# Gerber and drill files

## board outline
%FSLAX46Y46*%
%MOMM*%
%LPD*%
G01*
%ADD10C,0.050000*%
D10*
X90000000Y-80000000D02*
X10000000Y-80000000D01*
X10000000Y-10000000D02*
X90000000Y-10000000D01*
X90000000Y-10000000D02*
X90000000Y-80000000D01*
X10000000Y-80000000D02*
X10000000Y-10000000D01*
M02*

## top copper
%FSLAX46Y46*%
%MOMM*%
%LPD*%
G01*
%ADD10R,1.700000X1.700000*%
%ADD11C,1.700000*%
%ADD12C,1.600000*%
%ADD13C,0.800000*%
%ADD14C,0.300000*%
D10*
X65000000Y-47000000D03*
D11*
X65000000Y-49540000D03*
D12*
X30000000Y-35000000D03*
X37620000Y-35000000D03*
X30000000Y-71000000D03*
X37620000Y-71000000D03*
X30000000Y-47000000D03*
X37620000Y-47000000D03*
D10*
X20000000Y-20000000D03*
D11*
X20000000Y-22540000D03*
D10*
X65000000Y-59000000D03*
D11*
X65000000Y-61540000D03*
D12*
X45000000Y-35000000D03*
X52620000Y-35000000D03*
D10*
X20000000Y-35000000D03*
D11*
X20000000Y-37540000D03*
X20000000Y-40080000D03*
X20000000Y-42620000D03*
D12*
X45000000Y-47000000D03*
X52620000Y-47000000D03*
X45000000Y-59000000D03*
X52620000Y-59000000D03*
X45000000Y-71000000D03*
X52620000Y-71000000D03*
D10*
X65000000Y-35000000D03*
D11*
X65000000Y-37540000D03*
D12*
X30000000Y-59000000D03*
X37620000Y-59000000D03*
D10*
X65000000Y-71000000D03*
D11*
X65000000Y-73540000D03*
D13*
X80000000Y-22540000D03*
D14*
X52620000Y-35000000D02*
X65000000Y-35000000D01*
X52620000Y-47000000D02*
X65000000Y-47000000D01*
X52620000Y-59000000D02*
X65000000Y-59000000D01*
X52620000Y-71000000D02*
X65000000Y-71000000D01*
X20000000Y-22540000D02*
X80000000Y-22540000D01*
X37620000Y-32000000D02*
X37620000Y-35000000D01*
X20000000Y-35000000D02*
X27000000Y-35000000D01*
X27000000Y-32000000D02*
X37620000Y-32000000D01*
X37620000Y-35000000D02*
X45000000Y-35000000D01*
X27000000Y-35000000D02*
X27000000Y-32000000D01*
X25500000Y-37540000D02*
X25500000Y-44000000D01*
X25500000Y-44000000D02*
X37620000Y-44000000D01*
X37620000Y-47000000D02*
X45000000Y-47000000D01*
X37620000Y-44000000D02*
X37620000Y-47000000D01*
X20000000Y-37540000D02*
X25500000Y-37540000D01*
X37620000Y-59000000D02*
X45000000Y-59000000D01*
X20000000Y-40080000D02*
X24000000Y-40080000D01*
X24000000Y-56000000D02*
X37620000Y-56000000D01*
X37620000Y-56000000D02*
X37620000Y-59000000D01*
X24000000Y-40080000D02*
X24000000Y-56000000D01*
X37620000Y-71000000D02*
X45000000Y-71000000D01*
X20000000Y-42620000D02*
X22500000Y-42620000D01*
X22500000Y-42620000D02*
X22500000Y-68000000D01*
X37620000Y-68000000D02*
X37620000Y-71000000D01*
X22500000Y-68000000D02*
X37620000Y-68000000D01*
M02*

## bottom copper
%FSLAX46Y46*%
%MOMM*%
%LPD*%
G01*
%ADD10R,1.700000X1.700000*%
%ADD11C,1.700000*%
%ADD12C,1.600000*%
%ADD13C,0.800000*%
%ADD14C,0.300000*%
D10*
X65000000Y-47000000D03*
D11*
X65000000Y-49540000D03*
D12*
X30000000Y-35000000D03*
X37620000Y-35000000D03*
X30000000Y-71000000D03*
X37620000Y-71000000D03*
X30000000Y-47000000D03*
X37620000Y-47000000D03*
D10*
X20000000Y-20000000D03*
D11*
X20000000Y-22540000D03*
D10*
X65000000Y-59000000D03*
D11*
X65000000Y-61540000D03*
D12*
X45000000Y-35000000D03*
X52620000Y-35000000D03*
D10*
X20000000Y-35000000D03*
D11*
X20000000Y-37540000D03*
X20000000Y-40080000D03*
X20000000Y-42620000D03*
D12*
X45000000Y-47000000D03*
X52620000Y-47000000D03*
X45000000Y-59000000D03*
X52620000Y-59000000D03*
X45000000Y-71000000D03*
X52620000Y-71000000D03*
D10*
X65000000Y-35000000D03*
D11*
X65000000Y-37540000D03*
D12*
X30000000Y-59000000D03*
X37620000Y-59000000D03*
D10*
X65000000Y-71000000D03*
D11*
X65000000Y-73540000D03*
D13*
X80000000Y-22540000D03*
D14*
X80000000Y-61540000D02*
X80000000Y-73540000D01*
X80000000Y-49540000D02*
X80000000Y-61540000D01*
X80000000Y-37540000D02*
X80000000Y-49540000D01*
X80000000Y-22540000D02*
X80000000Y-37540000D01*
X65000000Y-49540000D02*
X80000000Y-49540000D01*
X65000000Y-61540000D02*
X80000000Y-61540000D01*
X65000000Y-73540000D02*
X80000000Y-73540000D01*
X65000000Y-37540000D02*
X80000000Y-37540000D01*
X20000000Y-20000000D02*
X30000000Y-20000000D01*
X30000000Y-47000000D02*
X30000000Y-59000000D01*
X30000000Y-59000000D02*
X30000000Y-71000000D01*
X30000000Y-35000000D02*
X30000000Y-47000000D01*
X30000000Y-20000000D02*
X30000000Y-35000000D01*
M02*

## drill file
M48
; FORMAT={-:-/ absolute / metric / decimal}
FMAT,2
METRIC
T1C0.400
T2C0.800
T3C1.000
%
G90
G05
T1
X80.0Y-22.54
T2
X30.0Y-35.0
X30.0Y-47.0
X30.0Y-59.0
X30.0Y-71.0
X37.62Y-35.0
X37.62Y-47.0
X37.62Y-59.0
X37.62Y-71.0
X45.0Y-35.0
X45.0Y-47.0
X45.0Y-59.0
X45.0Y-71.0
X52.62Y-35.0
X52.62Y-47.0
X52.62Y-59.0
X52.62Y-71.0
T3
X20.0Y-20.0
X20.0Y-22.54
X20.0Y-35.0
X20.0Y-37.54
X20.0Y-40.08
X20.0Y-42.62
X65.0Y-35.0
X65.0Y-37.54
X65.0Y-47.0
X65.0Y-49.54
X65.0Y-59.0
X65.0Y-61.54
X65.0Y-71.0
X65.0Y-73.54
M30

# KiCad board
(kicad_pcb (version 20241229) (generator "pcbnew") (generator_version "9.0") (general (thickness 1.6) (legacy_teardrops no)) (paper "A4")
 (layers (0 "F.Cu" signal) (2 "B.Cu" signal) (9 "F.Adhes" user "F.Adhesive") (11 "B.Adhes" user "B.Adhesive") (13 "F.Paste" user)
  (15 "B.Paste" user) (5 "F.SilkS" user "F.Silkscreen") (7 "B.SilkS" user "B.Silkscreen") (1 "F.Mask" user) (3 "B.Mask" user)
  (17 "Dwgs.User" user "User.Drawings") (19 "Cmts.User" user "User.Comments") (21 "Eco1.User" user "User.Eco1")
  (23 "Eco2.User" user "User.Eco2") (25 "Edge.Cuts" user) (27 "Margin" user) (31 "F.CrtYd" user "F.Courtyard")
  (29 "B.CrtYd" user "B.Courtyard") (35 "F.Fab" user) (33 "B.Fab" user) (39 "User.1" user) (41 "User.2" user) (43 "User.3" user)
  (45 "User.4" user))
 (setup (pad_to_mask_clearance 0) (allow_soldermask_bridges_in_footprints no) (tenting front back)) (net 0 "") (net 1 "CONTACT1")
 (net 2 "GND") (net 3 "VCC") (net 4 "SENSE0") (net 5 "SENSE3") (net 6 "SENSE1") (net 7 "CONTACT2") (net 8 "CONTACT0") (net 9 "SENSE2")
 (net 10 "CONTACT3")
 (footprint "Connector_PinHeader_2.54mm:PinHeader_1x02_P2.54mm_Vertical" (layer "F.Cu") (at 65 47)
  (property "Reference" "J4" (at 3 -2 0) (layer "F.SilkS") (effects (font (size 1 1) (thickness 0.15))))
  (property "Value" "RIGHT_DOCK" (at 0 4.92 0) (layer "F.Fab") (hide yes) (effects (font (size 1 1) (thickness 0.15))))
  (pad "1" thru_hole rect (at 0 0) (size 1.7 1.7) (drill 1) (layers "*.Cu" "*.Mask") (remove_unused_layers no) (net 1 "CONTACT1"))
  (pad "2" thru_hole circle (at 0 2.54) (size 1.7 1.7) (drill 1) (layers "*.Cu" "*.Mask") (remove_unused_layers no) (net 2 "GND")))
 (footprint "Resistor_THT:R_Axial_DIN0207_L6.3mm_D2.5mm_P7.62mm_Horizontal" (layer "F.Cu") (at 30 35)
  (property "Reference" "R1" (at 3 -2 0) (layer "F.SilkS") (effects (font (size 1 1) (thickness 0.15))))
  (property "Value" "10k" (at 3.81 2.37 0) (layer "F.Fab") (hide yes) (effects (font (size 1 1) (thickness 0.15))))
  (pad "1" thru_hole circle (at 0 0) (size 1.6 1.6) (drill 0.8) (layers "*.Cu" "*.Mask") (remove_unused_layers no) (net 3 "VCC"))
  (pad "2" thru_hole circle (at 7.62 0) (size 1.6 1.6) (drill 0.8) (layers "*.Cu" "*.Mask") (remove_unused_layers no) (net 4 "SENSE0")))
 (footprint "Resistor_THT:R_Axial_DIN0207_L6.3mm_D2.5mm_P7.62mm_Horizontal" (layer "F.Cu") (at 30 71)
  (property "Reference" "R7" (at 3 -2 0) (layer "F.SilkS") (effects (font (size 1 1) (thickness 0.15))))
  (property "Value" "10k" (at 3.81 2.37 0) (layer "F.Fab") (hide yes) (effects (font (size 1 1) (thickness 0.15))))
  (pad "1" thru_hole circle (at 0 0) (size 1.6 1.6) (drill 0.8) (layers "*.Cu" "*.Mask") (remove_unused_layers no) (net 3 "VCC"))
  (pad "2" thru_hole circle (at 7.62 0) (size 1.6 1.6) (drill 0.8) (layers "*.Cu" "*.Mask") (remove_unused_layers no) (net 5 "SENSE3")))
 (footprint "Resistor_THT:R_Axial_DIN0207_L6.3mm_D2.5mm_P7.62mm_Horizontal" (layer "F.Cu") (at 30 47)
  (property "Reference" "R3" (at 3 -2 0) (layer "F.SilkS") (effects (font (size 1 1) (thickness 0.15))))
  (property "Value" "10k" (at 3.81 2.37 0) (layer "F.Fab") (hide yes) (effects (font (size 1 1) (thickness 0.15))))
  (pad "1" thru_hole circle (at 0 0) (size 1.6 1.6) (drill 0.8) (layers "*.Cu" "*.Mask") (remove_unused_layers no) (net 3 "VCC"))
  (pad "2" thru_hole circle (at 7.62 0) (size 1.6 1.6) (drill 0.8) (layers "*.Cu" "*.Mask") (remove_unused_layers no) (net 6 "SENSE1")))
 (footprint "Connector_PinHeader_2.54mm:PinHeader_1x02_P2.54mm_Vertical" (layer "F.Cu") (at 20 20)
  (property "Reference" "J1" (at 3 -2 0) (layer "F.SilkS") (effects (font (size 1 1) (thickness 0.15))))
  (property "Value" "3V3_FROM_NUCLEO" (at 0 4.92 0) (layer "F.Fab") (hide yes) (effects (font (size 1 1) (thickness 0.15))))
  (pad "1" thru_hole rect (at 0 0) (size 1.7 1.7) (drill 1) (layers "*.Cu" "*.Mask") (remove_unused_layers no) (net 3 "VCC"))
  (pad "2" thru_hole circle (at 0 2.54) (size 1.7 1.7) (drill 1) (layers "*.Cu" "*.Mask") (remove_unused_layers no) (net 2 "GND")))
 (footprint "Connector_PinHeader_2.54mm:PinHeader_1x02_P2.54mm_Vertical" (layer "F.Cu") (at 65 59)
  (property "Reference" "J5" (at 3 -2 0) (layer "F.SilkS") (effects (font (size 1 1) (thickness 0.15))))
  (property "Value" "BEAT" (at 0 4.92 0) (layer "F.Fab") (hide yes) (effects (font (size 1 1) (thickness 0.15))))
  (pad "1" thru_hole rect (at 0 0) (size 1.7 1.7) (drill 1) (layers "*.Cu" "*.Mask") (remove_unused_layers no) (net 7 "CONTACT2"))
  (pad "2" thru_hole circle (at 0 2.54) (size 1.7 1.7) (drill 1) (layers "*.Cu" "*.Mask") (remove_unused_layers no) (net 2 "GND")))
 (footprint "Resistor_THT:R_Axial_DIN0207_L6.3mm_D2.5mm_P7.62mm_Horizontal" (layer "F.Cu") (at 45 35)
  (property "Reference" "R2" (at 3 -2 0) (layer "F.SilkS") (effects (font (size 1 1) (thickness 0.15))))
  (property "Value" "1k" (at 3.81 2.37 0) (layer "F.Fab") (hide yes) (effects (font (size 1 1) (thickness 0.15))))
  (pad "1" thru_hole circle (at 0 0) (size 1.6 1.6) (drill 0.8) (layers "*.Cu" "*.Mask") (remove_unused_layers no) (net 4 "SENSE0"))
  (pad "2" thru_hole circle (at 7.62 0) (size 1.6 1.6) (drill 0.8) (layers "*.Cu" "*.Mask") (remove_unused_layers no) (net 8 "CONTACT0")))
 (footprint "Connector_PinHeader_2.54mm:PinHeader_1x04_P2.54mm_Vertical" (layer "F.Cu") (at 20 35)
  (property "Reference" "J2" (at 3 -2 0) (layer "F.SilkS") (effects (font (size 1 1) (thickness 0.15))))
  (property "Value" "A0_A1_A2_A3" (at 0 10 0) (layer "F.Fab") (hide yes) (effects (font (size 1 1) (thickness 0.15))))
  (pad "1" thru_hole rect (at 0 0) (size 1.7 1.7) (drill 1) (layers "*.Cu" "*.Mask") (remove_unused_layers no) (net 4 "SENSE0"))
  (pad "2" thru_hole circle (at 0 2.54) (size 1.7 1.7) (drill 1) (layers "*.Cu" "*.Mask") (remove_unused_layers no) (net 6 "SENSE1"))
  (pad "3" thru_hole circle (at 0 5.08) (size 1.7 1.7) (drill 1) (layers "*.Cu" "*.Mask") (remove_unused_layers no) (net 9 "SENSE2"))
  (pad "4" thru_hole circle (at 0 7.62) (size 1.7 1.7) (drill 1) (layers "*.Cu" "*.Mask") (remove_unused_layers no) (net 5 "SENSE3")))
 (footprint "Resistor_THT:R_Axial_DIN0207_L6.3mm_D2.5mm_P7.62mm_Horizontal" (layer "F.Cu") (at 45 47)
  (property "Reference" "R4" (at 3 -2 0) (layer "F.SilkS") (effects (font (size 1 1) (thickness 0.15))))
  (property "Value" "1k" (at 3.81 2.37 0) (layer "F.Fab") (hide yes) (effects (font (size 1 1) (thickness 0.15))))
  (pad "1" thru_hole circle (at 0 0) (size 1.6 1.6) (drill 0.8) (layers "*.Cu" "*.Mask") (remove_unused_layers no) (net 6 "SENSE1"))
  (pad "2" thru_hole circle (at 7.62 0) (size 1.6 1.6) (drill 0.8) (layers "*.Cu" "*.Mask") (remove_unused_layers no) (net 1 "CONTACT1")))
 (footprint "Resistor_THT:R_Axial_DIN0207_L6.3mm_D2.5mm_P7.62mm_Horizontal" (layer "F.Cu") (at 45 59)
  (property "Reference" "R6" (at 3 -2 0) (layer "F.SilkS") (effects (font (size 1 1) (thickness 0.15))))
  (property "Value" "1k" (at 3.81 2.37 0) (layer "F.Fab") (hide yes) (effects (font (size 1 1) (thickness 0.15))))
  (pad "1" thru_hole circle (at 0 0) (size 1.6 1.6) (drill 0.8) (layers "*.Cu" "*.Mask") (remove_unused_layers no) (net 9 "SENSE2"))
  (pad "2" thru_hole circle (at 7.62 0) (size 1.6 1.6) (drill 0.8) (layers "*.Cu" "*.Mask") (remove_unused_layers no) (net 7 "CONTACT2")))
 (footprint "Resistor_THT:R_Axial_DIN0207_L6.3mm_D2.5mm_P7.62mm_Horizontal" (layer "F.Cu") (at 45 71)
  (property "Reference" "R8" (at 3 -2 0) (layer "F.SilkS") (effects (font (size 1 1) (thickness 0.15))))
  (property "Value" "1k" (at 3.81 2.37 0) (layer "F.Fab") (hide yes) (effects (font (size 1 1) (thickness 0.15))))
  (pad "1" thru_hole circle (at 0 0) (size 1.6 1.6) (drill 0.8) (layers "*.Cu" "*.Mask") (remove_unused_layers no) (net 5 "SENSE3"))
  (pad "2" thru_hole circle (at 7.62 0) (size 1.6 1.6) (drill 0.8) (layers "*.Cu" "*.Mask") (remove_unused_layers no) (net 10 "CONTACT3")))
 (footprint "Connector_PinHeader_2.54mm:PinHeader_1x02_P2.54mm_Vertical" (layer "F.Cu") (at 65 35)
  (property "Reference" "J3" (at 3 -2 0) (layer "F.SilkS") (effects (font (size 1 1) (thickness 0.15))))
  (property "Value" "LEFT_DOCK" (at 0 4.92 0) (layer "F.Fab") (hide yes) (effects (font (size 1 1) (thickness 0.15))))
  (pad "1" thru_hole rect (at 0 0) (size 1.7 1.7) (drill 1) (layers "*.Cu" "*.Mask") (remove_unused_layers no) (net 8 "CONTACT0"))
  (pad "2" thru_hole circle (at 0 2.54) (size 1.7 1.7) (drill 1) (layers "*.Cu" "*.Mask") (remove_unused_layers no) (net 2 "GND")))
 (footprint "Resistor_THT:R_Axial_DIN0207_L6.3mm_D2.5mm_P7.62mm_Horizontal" (layer "F.Cu") (at 30 59)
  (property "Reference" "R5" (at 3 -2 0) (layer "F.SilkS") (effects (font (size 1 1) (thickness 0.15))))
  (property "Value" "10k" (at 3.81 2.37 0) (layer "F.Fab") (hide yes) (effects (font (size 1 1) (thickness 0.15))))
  (pad "1" thru_hole circle (at 0 0) (size 1.6 1.6) (drill 0.8) (layers "*.Cu" "*.Mask") (remove_unused_layers no) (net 3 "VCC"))
  (pad "2" thru_hole circle (at 7.62 0) (size 1.6 1.6) (drill 0.8) (layers "*.Cu" "*.Mask") (remove_unused_layers no) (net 9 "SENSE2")))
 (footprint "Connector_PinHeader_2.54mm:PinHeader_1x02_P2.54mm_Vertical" (layer "F.Cu") (at 65 71)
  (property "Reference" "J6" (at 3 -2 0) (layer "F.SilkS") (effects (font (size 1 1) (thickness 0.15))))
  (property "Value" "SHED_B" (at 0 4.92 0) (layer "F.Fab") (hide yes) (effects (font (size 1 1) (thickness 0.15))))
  (pad "1" thru_hole rect (at 0 0) (size 1.7 1.7) (drill 1) (layers "*.Cu" "*.Mask") (remove_unused_layers no) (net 10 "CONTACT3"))
  (pad "2" thru_hole circle (at 0 2.54) (size 1.7 1.7) (drill 1) (layers "*.Cu" "*.Mask") (remove_unused_layers no) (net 2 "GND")))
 (gr_line (start 90 80) (end 10 80) (stroke (width 0.05) (type default)) (layer "Edge.Cuts"))
 (gr_line (start 10 10) (end 90 10) (stroke (width 0.05) (type default)) (layer "Edge.Cuts"))
 (gr_line (start 90 10) (end 90 80) (stroke (width 0.05) (type default)) (layer "Edge.Cuts"))
 (gr_line (start 10 80) (end 10 10) (stroke (width 0.05) (type default)) (layer "Edge.Cuts"))
 (segment (start 52.62 35) (end 65 35) (width 0.3) (layer "F.Cu") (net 8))
 (segment (start 52.62 47) (end 65 47) (width 0.3) (layer "F.Cu") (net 1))
 (segment (start 52.62 59) (end 65 59) (width 0.3) (layer "F.Cu") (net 7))
 (segment (start 52.62 71) (end 65 71) (width 0.3) (layer "F.Cu") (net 10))
 (segment (start 20 22.54) (end 80 22.54) (width 0.3) (layer "F.Cu") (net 2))
 (via (at 80 22.54) (size 0.8) (drill 0.4) (layers "F.Cu" "B.Cu") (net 2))
 (segment (start 80 61.54) (end 80 73.54) (width 0.3) (layer "B.Cu") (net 2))
 (segment (start 80 49.54) (end 80 61.54) (width 0.3) (layer "B.Cu") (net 2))
 (segment (start 80 37.54) (end 80 49.54) (width 0.3) (layer "B.Cu") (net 2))
 (segment (start 80 22.54) (end 80 37.54) (width 0.3) (layer "B.Cu") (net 2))
 (segment (start 65 49.54) (end 80 49.54) (width 0.3) (layer "B.Cu") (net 2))
 (segment (start 65 61.54) (end 80 61.54) (width 0.3) (layer "B.Cu") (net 2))
 (segment (start 65 73.54) (end 80 73.54) (width 0.3) (layer "B.Cu") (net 2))
 (segment (start 65 37.54) (end 80 37.54) (width 0.3) (layer "B.Cu") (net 2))
 (segment (start 37.62 32) (end 37.62 35) (width 0.3) (layer "F.Cu") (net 4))
 (segment (start 20 35) (end 27 35) (width 0.3) (layer "F.Cu") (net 4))
 (segment (start 27 32) (end 37.62 32) (width 0.3) (layer "F.Cu") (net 4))
 (segment (start 37.62 35) (end 45 35) (width 0.3) (layer "F.Cu") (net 4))
 (segment (start 27 35) (end 27 32) (width 0.3) (layer "F.Cu") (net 4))
 (segment (start 25.5 37.54) (end 25.5 44) (width 0.3) (layer "F.Cu") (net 6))
 (segment (start 25.5 44) (end 37.62 44) (width 0.3) (layer "F.Cu") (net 6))
 (segment (start 37.62 47) (end 45 47) (width 0.3) (layer "F.Cu") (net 6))
 (segment (start 37.62 44) (end 37.62 47) (width 0.3) (layer "F.Cu") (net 6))
 (segment (start 20 37.54) (end 25.5 37.54) (width 0.3) (layer "F.Cu") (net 6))
 (segment (start 37.62 59) (end 45 59) (width 0.3) (layer "F.Cu") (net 9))
 (segment (start 20 40.08) (end 24 40.08) (width 0.3) (layer "F.Cu") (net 9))
 (segment (start 24 56) (end 37.62 56) (width 0.3) (layer "F.Cu") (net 9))
 (segment (start 37.62 56) (end 37.62 59) (width 0.3) (layer "F.Cu") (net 9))
 (segment (start 24 40.08) (end 24 56) (width 0.3) (layer "F.Cu") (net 9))
 (segment (start 37.62 71) (end 45 71) (width 0.3) (layer "F.Cu") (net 5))
 (segment (start 20 42.62) (end 22.5 42.62) (width 0.3) (layer "F.Cu") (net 5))
 (segment (start 22.5 42.62) (end 22.5 68) (width 0.3) (layer "F.Cu") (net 5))
 (segment (start 37.62 68) (end 37.62 71) (width 0.3) (layer "F.Cu") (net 5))
 (segment (start 22.5 68) (end 37.62 68) (width 0.3) (layer "F.Cu") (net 5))
 (segment (start 20 20) (end 30 20) (width 0.3) (layer "B.Cu") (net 3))
 (segment (start 30 47) (end 30 59) (width 0.3) (layer "B.Cu") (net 3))
 (segment (start 30 59) (end 30 71) (width 0.3) (layer "B.Cu") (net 3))
 (segment (start 30 35) (end 30 47) (width 0.3) (layer "B.Cu") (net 3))
 (segment (start 30 20) (end 30 35) (width 0.3) (layer "B.Cu") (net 3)))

